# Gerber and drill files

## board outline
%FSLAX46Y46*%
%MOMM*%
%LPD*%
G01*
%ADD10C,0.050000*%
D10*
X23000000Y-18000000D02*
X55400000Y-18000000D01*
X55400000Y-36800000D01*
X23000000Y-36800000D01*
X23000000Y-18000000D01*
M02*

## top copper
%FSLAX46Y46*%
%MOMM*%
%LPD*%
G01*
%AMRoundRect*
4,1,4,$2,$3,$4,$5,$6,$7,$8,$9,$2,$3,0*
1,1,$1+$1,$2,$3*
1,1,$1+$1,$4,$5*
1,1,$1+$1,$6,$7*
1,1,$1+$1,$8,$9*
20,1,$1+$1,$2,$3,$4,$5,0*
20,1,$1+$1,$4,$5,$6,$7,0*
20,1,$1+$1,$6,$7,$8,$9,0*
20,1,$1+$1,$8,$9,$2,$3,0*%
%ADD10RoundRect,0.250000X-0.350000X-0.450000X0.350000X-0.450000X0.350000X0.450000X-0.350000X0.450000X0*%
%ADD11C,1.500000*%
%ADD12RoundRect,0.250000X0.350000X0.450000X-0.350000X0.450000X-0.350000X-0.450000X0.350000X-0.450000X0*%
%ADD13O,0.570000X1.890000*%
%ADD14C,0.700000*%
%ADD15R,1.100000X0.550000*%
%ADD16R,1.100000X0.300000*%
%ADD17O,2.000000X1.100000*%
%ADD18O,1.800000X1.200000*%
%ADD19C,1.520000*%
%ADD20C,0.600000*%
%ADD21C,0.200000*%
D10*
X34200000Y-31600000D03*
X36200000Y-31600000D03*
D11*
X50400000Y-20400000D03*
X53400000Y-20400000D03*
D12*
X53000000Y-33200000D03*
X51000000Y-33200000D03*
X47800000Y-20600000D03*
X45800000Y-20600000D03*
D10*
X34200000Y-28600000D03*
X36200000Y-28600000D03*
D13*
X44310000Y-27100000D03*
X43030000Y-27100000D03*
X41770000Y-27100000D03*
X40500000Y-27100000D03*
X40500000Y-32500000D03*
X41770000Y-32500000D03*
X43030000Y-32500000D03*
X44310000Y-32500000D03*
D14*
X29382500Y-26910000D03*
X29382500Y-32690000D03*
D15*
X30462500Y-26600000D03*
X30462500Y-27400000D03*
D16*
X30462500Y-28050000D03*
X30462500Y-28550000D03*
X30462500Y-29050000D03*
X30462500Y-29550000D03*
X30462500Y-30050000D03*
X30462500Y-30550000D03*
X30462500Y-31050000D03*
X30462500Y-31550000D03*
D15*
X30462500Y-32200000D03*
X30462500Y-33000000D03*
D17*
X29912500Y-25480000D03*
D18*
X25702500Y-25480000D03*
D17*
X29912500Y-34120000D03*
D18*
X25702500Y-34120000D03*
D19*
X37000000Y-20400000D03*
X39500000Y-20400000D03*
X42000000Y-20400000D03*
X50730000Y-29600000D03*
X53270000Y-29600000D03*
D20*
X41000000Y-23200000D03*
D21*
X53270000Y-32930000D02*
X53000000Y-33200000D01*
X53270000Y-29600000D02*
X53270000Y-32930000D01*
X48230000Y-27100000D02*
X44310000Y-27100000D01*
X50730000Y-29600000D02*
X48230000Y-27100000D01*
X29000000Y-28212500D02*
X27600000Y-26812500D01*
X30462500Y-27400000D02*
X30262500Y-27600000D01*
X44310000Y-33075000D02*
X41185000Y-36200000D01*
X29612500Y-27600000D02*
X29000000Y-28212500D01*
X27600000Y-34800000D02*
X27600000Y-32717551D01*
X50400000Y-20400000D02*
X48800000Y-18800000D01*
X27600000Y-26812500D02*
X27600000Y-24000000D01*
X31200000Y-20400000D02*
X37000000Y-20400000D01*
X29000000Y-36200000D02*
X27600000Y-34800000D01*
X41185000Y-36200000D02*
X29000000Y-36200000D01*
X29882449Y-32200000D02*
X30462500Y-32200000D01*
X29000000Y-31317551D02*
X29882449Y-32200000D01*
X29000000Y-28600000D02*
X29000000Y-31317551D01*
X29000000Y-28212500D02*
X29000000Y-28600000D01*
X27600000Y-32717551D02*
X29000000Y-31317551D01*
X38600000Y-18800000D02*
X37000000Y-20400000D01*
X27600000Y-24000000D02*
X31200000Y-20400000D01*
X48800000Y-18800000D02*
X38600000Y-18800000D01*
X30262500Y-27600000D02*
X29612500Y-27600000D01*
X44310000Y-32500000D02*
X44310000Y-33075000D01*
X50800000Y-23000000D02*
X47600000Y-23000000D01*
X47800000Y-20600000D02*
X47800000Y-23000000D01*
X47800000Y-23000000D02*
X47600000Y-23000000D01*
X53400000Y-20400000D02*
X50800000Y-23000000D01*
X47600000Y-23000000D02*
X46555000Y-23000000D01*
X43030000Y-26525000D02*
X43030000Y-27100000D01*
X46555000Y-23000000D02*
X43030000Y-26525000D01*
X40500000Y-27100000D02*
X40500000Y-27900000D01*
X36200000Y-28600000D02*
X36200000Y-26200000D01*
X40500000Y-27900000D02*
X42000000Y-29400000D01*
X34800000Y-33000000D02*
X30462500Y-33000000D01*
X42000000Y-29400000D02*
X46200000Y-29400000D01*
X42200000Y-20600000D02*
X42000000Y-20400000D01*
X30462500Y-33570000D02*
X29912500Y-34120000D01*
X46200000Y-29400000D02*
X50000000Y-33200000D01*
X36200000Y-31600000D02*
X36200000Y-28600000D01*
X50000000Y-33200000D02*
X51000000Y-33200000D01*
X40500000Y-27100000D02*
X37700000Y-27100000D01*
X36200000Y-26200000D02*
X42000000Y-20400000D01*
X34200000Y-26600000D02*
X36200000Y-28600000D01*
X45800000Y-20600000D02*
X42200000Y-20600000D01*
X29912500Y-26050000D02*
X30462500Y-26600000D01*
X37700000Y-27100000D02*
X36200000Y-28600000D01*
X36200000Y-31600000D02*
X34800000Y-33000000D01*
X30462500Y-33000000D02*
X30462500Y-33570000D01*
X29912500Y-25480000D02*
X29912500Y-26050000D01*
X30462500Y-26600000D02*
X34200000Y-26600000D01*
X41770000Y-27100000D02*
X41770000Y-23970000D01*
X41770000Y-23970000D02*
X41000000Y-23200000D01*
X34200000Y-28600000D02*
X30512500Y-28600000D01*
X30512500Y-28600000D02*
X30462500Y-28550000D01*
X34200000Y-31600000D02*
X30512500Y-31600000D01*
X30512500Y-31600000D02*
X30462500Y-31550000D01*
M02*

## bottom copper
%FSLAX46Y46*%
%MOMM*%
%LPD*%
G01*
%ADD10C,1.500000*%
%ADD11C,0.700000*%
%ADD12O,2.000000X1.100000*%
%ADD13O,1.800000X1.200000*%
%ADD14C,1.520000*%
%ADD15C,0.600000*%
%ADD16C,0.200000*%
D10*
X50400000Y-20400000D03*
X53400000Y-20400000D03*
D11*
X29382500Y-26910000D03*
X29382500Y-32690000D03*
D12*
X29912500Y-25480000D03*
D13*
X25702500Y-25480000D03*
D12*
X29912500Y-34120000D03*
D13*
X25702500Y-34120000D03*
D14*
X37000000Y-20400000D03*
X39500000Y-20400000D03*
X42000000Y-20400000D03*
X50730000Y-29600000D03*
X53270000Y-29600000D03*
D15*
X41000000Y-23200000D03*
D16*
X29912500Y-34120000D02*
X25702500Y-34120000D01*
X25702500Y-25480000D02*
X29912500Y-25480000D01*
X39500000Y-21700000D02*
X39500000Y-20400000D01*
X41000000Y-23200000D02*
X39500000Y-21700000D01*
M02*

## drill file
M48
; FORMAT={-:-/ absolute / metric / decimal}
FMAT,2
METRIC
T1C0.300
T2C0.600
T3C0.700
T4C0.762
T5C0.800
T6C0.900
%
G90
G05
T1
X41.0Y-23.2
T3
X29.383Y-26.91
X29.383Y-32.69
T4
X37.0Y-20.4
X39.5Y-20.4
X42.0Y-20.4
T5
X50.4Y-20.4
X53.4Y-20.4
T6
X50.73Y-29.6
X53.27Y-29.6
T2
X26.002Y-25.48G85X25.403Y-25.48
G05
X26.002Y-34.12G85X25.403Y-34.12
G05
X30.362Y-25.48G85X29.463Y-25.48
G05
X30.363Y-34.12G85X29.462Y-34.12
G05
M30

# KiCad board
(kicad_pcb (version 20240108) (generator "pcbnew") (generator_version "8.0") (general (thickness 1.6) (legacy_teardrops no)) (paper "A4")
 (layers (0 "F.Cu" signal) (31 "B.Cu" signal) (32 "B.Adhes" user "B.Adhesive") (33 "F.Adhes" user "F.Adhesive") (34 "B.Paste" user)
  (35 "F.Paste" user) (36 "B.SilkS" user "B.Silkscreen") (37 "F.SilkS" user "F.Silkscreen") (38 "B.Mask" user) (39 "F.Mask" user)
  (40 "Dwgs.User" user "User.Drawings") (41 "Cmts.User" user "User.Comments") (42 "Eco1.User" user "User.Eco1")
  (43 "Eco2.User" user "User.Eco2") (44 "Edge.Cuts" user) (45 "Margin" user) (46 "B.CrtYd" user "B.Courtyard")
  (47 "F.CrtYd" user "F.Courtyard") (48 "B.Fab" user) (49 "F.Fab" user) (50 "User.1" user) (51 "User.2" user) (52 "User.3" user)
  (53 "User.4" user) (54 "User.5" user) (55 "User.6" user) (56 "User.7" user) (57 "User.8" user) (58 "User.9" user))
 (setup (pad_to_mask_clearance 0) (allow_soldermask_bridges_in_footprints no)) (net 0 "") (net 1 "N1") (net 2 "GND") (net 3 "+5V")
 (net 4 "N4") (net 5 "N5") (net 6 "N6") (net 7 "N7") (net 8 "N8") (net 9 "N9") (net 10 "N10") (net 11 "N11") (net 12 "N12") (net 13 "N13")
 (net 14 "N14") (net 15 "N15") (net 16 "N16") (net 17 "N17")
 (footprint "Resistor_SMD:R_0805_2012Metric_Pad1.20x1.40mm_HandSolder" (layer "F.Cu") (at 35.2 31.6)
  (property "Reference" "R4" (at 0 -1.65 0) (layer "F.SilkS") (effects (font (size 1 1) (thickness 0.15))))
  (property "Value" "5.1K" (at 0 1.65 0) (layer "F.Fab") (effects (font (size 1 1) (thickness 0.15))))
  (pad "1" smd roundrect (at -1 0) (size 1.2 1.4) (layers "F.Cu" "F.Paste" "F.Mask") (roundrect_rratio 0.208333) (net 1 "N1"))
  (pad "2" smd roundrect (at 1 0) (size 1.2 1.4) (layers "F.Cu" "F.Paste" "F.Mask") (roundrect_rratio 0.208333) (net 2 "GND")))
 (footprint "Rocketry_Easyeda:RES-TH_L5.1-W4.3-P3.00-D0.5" (layer "F.Cu") (at 51.9 20.4)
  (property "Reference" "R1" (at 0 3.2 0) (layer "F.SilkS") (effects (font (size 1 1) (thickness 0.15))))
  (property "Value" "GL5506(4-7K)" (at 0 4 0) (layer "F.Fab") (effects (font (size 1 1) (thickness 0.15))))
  (pad "1" thru_hole circle (at -1.5 0) (size 1.5 1.5) (drill 0.799998) (layers "*.Cu" "*.Mask") (remove_unused_layers no) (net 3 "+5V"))
  (pad "2" thru_hole circle (at 1.5 0) (size 1.5 1.5) (drill 0.799998) (layers "*.Cu" "*.Mask") (remove_unused_layers no) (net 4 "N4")))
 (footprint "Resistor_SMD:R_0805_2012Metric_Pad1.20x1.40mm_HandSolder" (layer "F.Cu") (at 52 33.2 180)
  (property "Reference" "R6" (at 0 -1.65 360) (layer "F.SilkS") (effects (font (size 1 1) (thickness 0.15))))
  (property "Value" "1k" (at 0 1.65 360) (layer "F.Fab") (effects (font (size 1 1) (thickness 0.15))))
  (pad "1" smd roundrect (at -1 0 180) (size 1.2 1.4) (layers "F.Cu" "F.Paste" "F.Mask") (roundrect_rratio 0.208333) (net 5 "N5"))
  (pad "2" smd roundrect (at 1 0 180) (size 1.2 1.4) (layers "F.Cu" "F.Paste" "F.Mask") (roundrect_rratio 0.208333) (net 2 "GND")))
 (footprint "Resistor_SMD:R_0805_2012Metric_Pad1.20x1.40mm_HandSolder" (layer "F.Cu") (at 46.8 20.6 180)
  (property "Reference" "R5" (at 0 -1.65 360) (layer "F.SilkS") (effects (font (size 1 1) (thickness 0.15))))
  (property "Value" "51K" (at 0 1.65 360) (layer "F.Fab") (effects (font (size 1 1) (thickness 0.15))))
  (pad "1" smd roundrect (at -1 0 180) (size 1.2 1.4) (layers "F.Cu" "F.Paste" "F.Mask") (roundrect_rratio 0.208333) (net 4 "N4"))
  (pad "2" smd roundrect (at 1 0 180) (size 1.2 1.4) (layers "F.Cu" "F.Paste" "F.Mask") (roundrect_rratio 0.208333) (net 2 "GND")))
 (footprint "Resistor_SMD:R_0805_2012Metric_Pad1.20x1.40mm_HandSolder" (layer "F.Cu") (at 35.2 28.6)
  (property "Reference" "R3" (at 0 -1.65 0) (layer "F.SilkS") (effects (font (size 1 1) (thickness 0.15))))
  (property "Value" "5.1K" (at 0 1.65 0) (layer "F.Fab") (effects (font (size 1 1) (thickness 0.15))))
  (pad "1" smd roundrect (at -1 0) (size 1.2 1.4) (layers "F.Cu" "F.Paste" "F.Mask") (roundrect_rratio 0.208333) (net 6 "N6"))
  (pad "2" smd roundrect (at 1 0) (size 1.2 1.4) (layers "F.Cu" "F.Paste" "F.Mask") (roundrect_rratio 0.208333) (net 2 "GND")))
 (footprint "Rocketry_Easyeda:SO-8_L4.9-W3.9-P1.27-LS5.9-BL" (layer "F.Cu") (at 42.4 29.8 180)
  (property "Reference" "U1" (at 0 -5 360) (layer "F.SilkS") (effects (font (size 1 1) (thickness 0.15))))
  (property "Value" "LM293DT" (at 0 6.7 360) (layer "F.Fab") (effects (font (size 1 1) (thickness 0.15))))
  (pad "1" smd oval (at -1.91 2.7 180) (size 0.57 1.89) (layers "F.Cu" "F.Paste" "F.Mask") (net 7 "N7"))
  (pad "2" smd oval (at -0.63 2.7 180) (size 0.57 1.89) (layers "F.Cu" "F.Paste" "F.Mask") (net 4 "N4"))
  (pad "3" smd oval (at 0.63 2.7 180) (size 0.57 1.89) (layers "F.Cu" "F.Paste" "F.Mask") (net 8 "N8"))
  (pad "4" smd oval (at 1.9 2.7 180) (size 0.57 1.89) (layers "F.Cu" "F.Paste" "F.Mask") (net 2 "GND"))
  (pad "5" smd oval (at 1.9 -2.7 180) (size 0.57 1.89) (layers "F.Cu" "F.Paste" "F.Mask") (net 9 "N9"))
  (pad "6" smd oval (at 0.63 -2.7 180) (size 0.57 1.89) (layers "F.Cu" "F.Paste" "F.Mask") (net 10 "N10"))
  (pad "7" smd oval (at -0.63 -2.7 180) (size 0.57 1.89) (layers "F.Cu" "F.Paste" "F.Mask") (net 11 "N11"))
  (pad "8" smd oval (at -1.91 -2.7 180) (size 0.57 1.89) (layers "F.Cu" "F.Paste" "F.Mask") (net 3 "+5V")))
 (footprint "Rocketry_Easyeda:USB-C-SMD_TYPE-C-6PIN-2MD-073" (layer "F.Cu") (at 28.0825 29.8 -90)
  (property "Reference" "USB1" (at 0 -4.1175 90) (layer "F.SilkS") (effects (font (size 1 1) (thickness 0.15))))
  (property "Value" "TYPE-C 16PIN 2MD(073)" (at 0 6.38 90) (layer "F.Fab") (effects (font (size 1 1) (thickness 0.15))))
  (pad "" thru_hole circle (at -2.89 -1.3 270) (size 0.7 0.7) (drill 0.7) (layers "*.Cu" "*.Mask") (remove_unused_layers no))
  (pad "" thru_hole circle (at 2.89 -1.3 270) (size 0.7 0.7) (drill 0.7) (layers "*.Cu" "*.Mask") (remove_unused_layers no))
  (pad "1" smd rect (at -3.2 -2.38 270) (size 0.55 1.1) (layers "F.Cu" "F.Paste" "F.Mask") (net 2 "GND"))
  (pad "2" smd rect (at -2.4 -2.38 270) (size 0.55 1.1) (layers "F.Cu" "F.Paste" "F.Mask") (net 3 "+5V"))
  (pad "3" smd rect (at -1.75 -2.38 270) (size 0.3 1.1) (layers "F.Cu" "F.Paste" "F.Mask") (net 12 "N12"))
  (pad "4" smd rect (at -1.25 -2.38 270) (size 0.3 1.1) (layers "F.Cu" "F.Paste" "F.Mask") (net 6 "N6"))
  (pad "5" smd rect (at -0.75 -2.38 270) (size 0.3 1.1) (layers "F.Cu" "F.Paste" "F.Mask") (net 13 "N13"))
  (pad "6" smd rect (at -0.25 -2.38 270) (size 0.3 1.1) (layers "F.Cu" "F.Paste" "F.Mask") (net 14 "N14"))
  (pad "7" smd rect (at 0.25 -2.38 270) (size 0.3 1.1) (layers "F.Cu" "F.Paste" "F.Mask") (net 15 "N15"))
  (pad "8" smd rect (at 0.75 -2.38 270) (size 0.3 1.1) (layers "F.Cu" "F.Paste" "F.Mask") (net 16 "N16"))
  (pad "9" smd rect (at 1.25 -2.38 270) (size 0.3 1.1) (layers "F.Cu" "F.Paste" "F.Mask") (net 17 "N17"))
  (pad "10" smd rect (at 1.75 -2.38 270) (size 0.3 1.1) (layers "F.Cu" "F.Paste" "F.Mask") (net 1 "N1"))
  (pad "11" smd rect (at 2.4 -2.38 270) (size 0.55 1.1) (layers "F.Cu" "F.Paste" "F.Mask") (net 3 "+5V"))
  (pad "12" smd rect (at 3.2 -2.38 270) (size 0.55 1.1) (layers "F.Cu" "F.Paste" "F.Mask") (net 2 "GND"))
  (pad "13" thru_hole oval (at -4.32 -1.83 270) (size 1.1 2) (drill oval 0.599999 1.499997) (layers "*.Cu" "*.Mask")
   (remove_unused_layers no) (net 2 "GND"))
  (pad "13" thru_hole oval (at -4.32 2.38 270) (size 1.2 1.8) (drill oval 0.599999 1.199998) (layers "*.Cu" "*.Mask")
   (remove_unused_layers no) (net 2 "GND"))
  (pad "14" thru_hole oval (at 4.32 -1.83 270) (size 1.1 2) (drill oval 0.599999 1.500022) (layers "*.Cu" "*.Mask")
   (remove_unused_layers no) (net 2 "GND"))
  (pad "14" thru_hole oval (at 4.32 2.38 270) (size 1.2 1.8) (drill oval 0.599999 1.199998) (layers "*.Cu" "*.Mask")
   (remove_unused_layers no) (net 2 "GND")))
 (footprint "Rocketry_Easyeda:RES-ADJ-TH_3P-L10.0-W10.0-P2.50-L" (layer "F.Cu") (at 39.5 20.4)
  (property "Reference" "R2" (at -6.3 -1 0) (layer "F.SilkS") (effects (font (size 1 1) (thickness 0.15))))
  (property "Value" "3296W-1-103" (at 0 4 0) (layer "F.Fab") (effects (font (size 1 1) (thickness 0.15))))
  (pad "1" thru_hole circle (at -2.5 0) (size 1.52 1.52) (drill 0.762) (layers "*.Cu" "*.Mask") (remove_unused_layers no) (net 3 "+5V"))
  (pad "2" thru_hole circle (at 0 0) (size 1.52 1.52) (drill 0.762) (layers "*.Cu" "*.Mask") (remove_unused_layers no) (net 8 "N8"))
  (pad "3" thru_hole circle (at 2.5 0) (size 1.52 1.52) (drill 0.762) (layers "*.Cu" "*.Mask") (remove_unused_layers no) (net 2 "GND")))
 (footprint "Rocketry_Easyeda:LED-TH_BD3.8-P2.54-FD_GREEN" (layer "F.Cu") (at 52 29.6)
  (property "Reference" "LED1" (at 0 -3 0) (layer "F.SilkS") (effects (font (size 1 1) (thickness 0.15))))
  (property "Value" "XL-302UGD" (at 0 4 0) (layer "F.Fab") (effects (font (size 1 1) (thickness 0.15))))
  (pad "1" thru_hole circle (at -1.27 0) (size 1.52 1.52) (drill 0.900024) (layers "*.Cu" "*.Mask") (remove_unused_layers no) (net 7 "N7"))
  (pad "2" thru_hole circle (at 1.27 0) (size 1.52 1.52) (drill 0.900024) (layers "*.Cu" "*.Mask") (remove_unused_layers no) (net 5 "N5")))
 (gr_rect (start 23 18) (end 55.4 36.8) (stroke (width 0.05) (type default)) (fill none) (layer "Edge.Cuts"))
 (segment (start 53.27 32.93) (end 53 33.2) (width 0.2) (layer "F.Cu") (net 5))
 (segment (start 53.27 29.6) (end 53.27 32.93) (width 0.2) (layer "F.Cu") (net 5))
 (segment (start 48.23 27.1) (end 44.31 27.1) (width 0.2) (layer "F.Cu") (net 7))
 (segment (start 50.73 29.6) (end 48.23 27.1) (width 0.2) (layer "F.Cu") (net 7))
 (segment (start 29 28.2125) (end 27.6 26.8125) (width 0.2) (layer "F.Cu") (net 3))
 (segment (start 30.4625 27.4) (end 30.2625 27.6) (width 0.2) (layer "F.Cu") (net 3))
 (segment (start 44.31 33.075) (end 41.185 36.2) (width 0.2) (layer "F.Cu") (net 3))
 (segment (start 29.6125 27.6) (end 29 28.2125) (width 0.2) (layer "F.Cu") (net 3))
 (segment (start 27.6 34.8) (end 27.6 32.717551) (width 0.2) (layer "F.Cu") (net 3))
 (segment (start 50.4 20.4) (end 48.8 18.8) (width 0.2) (layer "F.Cu") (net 3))
 (segment (start 27.6 26.8125) (end 27.6 24) (width 0.2) (layer "F.Cu") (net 3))
 (segment (start 31.2 20.4) (end 37 20.4) (width 0.2) (layer "F.Cu") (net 3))
 (segment (start 29 36.2) (end 27.6 34.8) (width 0.2) (layer "F.Cu") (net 3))
 (segment (start 41.185 36.2) (end 29 36.2) (width 0.2) (layer "F.Cu") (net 3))
 (segment (start 29.882449 32.2) (end 30.4625 32.2) (width 0.2) (layer "F.Cu") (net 3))
 (segment (start 29 31.317551) (end 29.882449 32.2) (width 0.2) (layer "F.Cu") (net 3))
 (segment (start 29 28.6) (end 29 31.317551) (width 0.2) (layer "F.Cu") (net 3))
 (segment (start 29 28.2125) (end 29 28.6) (width 0.2) (layer "F.Cu") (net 3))
 (segment (start 27.6 32.717551) (end 29 31.317551) (width 0.2) (layer "F.Cu") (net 3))
 (segment (start 38.6 18.8) (end 37 20.4) (width 0.2) (layer "F.Cu") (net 3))
 (segment (start 27.6 24) (end 31.2 20.4) (width 0.2) (layer "F.Cu") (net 3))
 (segment (start 48.8 18.8) (end 38.6 18.8) (width 0.2) (layer "F.Cu") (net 3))
 (segment (start 30.2625 27.6) (end 29.6125 27.6) (width 0.2) (layer "F.Cu") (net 3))
 (segment (start 44.31 32.5) (end 44.31 33.075) (width 0.2) (layer "F.Cu") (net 3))
 (segment (start 50.8 23) (end 47.6 23) (width 0.2) (layer "F.Cu") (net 4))
 (segment (start 47.8 20.6) (end 47.8 23) (width 0.2) (layer "F.Cu") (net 4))
 (segment (start 47.8 23) (end 47.6 23) (width 0.2) (layer "F.Cu") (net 4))
 (segment (start 53.4 20.4) (end 50.8 23) (width 0.2) (layer "F.Cu") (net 4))
 (segment (start 47.6 23) (end 46.555 23) (width 0.2) (layer "F.Cu") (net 4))
 (segment (start 43.03 26.525) (end 43.03 27.1) (width 0.2) (layer "F.Cu") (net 4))
 (segment (start 46.555 23) (end 43.03 26.525) (width 0.2) (layer "F.Cu") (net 4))
 (segment (start 40.5 27.1) (end 40.5 27.9) (width 0.2) (layer "F.Cu") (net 2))
 (segment (start 36.2 28.6) (end 36.2 26.2) (width 0.2) (layer "F.Cu") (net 2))
 (segment (start 40.5 27.9) (end 42 29.4) (width 0.2) (layer "F.Cu") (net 2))
 (segment (start 34.8 33) (end 30.4625 33) (width 0.2) (layer "F.Cu") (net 2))
 (segment (start 42 29.4) (end 46.2 29.4) (width 0.2) (layer "F.Cu") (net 2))
 (segment (start 42.2 20.6) (end 42 20.4) (width 0.2) (layer "F.Cu") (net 2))
 (segment (start 30.4625 33.57) (end 29.9125 34.12) (width 0.2) (layer "F.Cu") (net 2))
 (segment (start 46.2 29.4) (end 50 33.2) (width 0.2) (layer "F.Cu") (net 2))
 (segment (start 36.2 31.6) (end 36.2 28.6) (width 0.2) (layer "F.Cu") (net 2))
 (segment (start 50 33.2) (end 51 33.2) (width 0.2) (layer "F.Cu") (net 2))
 (segment (start 40.5 27.1) (end 37.7 27.1) (width 0.2) (layer "F.Cu") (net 2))
 (segment (start 36.2 26.2) (end 42 20.4) (width 0.2) (layer "F.Cu") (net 2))
 (segment (start 34.2 26.6) (end 36.2 28.6) (width 0.2) (layer "F.Cu") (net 2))
 (segment (start 45.8 20.6) (end 42.2 20.6) (width 0.2) (layer "F.Cu") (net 2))
 (segment (start 29.9125 26.05) (end 30.4625 26.6) (width 0.2) (layer "F.Cu") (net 2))
 (segment (start 37.7 27.1) (end 36.2 28.6) (width 0.2) (layer "F.Cu") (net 2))
 (segment (start 36.2 31.6) (end 34.8 33) (width 0.2) (layer "F.Cu") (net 2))
 (segment (start 30.4625 33) (end 30.4625 33.57) (width 0.2) (layer "F.Cu") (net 2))
 (segment (start 29.9125 25.48) (end 29.9125 26.05) (width 0.2) (layer "F.Cu") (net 2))
 (segment (start 30.4625 26.6) (end 34.2 26.6) (width 0.2) (layer "F.Cu") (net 2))
 (segment (start 29.9125 34.12) (end 25.7025 34.12) (width 0.2) (layer "B.Cu") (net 2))
 (segment (start 25.7025 25.48) (end 29.9125 25.48) (width 0.2) (layer "B.Cu") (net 2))
 (segment (start 41.77 27.1) (end 41.77 23.97) (width 0.2) (layer "F.Cu") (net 8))
 (segment (start 41.77 23.97) (end 41 23.2) (width 0.2) (layer "F.Cu") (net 8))
 (via (at 41 23.2) (size 0.6) (drill 0.3) (layers "F.Cu" "B.Cu") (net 8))
 (segment (start 39.5 21.7) (end 39.5 20.4) (width 0.2) (layer "B.Cu") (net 8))
 (segment (start 41 23.2) (end 39.5 21.7) (width 0.2) (layer "B.Cu") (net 8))
 (segment (start 34.2 28.6) (end 30.5125 28.6) (width 0.2) (layer "F.Cu") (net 6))
 (segment (start 30.5125 28.6) (end 30.4625 28.55) (width 0.2) (layer "F.Cu") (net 6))
 (segment (start 34.2 31.6) (end 30.5125 31.6) (width 0.2) (layer "F.Cu") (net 1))
 (segment (start 30.5125 31.6) (end 30.4625 31.55) (width 0.2) (layer "F.Cu") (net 1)))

